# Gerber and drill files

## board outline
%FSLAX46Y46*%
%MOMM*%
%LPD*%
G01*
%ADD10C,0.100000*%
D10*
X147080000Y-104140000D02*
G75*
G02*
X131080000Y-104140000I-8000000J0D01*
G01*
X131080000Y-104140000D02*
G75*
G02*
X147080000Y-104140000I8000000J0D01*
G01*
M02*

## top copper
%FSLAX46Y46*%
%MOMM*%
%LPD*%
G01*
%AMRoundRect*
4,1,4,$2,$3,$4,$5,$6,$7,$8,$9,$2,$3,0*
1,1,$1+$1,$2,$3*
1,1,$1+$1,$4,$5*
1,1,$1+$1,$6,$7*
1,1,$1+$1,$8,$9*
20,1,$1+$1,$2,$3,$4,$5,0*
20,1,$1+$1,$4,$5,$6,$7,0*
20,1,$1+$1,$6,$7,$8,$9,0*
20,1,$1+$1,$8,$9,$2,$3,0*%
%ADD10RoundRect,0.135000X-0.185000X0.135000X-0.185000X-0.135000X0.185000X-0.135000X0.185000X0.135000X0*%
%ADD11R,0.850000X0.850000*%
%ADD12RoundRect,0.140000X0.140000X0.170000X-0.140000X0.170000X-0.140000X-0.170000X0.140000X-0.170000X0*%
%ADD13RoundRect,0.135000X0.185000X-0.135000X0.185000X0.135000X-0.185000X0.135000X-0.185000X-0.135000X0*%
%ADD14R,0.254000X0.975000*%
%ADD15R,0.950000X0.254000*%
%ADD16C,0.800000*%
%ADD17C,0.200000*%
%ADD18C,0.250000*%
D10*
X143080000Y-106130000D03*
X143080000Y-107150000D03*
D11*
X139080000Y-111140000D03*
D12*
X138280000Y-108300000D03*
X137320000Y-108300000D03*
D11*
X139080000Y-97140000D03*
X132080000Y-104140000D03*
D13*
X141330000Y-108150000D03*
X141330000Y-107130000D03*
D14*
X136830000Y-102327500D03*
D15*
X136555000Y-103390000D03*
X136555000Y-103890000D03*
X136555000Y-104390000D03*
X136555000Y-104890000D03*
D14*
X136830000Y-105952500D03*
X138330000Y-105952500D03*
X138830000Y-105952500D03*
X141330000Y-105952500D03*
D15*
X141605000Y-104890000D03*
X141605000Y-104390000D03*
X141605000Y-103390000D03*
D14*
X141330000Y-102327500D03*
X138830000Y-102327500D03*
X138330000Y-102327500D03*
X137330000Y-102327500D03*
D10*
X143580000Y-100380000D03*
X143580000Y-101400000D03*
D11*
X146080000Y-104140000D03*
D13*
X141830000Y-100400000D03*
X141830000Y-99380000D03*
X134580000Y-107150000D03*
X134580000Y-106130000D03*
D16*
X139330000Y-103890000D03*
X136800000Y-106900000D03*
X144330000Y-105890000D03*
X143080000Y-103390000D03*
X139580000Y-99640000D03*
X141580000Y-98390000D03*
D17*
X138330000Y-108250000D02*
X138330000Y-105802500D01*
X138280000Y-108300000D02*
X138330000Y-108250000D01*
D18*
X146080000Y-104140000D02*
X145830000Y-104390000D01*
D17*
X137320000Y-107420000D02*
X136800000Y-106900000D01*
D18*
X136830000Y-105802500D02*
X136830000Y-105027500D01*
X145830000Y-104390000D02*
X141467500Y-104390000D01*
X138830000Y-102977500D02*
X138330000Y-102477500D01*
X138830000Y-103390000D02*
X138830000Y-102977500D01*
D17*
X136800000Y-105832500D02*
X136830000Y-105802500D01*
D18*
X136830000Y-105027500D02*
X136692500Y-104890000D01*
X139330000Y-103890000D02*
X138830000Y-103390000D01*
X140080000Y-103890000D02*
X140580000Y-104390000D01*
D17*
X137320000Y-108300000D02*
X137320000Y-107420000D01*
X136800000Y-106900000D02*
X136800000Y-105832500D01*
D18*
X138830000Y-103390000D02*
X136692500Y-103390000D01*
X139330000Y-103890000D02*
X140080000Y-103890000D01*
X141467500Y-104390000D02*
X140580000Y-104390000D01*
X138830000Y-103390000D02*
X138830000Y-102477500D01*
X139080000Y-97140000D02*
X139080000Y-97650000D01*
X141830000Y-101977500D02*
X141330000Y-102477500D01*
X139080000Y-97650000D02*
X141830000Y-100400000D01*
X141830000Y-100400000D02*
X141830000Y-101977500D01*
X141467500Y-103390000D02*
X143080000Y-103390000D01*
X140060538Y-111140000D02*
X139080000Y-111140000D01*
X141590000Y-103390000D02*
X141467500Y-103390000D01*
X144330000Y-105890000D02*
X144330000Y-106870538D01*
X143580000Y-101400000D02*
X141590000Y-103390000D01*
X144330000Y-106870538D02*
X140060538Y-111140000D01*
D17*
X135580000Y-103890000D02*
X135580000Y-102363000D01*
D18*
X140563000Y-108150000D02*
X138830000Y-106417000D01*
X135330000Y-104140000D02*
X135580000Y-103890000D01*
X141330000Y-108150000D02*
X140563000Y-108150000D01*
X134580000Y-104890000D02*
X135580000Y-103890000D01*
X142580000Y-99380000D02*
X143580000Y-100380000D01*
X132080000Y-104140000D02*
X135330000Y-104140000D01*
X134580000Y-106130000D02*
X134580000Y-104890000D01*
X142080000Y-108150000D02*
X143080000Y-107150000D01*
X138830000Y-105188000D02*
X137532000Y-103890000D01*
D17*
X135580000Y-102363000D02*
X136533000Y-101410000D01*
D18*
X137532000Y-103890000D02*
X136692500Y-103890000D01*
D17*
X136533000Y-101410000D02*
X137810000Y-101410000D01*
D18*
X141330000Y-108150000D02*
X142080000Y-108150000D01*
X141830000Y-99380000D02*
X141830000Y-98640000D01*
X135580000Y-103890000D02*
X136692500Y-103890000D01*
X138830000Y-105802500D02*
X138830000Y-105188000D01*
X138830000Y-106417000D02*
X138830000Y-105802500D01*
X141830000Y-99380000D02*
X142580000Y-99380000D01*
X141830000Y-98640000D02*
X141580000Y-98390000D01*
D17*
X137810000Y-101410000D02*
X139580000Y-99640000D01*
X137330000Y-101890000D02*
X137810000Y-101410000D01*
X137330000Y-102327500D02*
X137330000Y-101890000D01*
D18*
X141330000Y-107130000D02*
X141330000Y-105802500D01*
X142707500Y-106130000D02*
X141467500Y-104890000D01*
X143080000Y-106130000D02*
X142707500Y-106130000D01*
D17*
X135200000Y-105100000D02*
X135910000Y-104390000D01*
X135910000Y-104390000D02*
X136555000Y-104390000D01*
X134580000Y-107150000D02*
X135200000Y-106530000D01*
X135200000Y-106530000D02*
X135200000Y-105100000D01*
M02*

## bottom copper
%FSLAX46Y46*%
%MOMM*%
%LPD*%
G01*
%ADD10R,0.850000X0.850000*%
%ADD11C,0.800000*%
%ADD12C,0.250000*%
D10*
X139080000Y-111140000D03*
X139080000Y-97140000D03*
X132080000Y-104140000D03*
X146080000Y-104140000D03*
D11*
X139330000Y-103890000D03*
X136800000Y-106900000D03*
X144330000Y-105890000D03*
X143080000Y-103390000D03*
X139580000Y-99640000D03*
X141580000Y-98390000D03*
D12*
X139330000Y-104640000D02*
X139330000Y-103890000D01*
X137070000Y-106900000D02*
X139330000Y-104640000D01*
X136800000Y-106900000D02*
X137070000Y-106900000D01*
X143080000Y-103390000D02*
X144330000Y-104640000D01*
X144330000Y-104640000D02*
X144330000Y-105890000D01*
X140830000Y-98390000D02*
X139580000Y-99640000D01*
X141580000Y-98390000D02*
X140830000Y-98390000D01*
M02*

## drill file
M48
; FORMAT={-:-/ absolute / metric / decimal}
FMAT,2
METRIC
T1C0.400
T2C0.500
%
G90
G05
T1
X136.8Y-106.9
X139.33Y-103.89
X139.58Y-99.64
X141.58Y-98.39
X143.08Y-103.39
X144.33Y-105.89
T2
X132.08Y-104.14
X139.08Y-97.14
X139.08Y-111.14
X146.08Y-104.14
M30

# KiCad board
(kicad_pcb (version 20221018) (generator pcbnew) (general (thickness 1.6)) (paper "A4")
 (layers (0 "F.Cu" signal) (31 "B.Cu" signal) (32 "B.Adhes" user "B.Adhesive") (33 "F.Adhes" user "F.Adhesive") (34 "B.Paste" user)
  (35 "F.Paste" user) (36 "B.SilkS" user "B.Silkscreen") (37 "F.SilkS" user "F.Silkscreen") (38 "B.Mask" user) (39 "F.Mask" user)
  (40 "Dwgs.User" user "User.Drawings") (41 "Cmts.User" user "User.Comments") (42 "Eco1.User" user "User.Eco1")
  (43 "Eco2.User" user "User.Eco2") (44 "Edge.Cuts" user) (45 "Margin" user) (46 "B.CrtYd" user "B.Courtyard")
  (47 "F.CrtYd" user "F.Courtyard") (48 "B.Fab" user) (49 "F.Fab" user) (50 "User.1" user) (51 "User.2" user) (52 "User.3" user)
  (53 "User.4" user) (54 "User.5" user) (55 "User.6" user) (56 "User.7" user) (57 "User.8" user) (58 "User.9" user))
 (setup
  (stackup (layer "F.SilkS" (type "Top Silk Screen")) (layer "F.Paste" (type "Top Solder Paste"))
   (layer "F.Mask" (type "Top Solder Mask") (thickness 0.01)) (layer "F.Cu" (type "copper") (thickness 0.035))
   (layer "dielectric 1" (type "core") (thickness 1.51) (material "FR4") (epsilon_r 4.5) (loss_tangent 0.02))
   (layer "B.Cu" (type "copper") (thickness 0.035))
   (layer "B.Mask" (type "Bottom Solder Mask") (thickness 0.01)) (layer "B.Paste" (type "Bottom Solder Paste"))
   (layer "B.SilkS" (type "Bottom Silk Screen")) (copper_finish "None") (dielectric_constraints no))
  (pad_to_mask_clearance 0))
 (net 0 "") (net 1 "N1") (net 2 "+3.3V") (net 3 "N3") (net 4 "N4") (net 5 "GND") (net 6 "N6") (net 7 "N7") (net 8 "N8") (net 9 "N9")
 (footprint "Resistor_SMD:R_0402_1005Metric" (layer "F.Cu") (at 143.08 106.64 -90)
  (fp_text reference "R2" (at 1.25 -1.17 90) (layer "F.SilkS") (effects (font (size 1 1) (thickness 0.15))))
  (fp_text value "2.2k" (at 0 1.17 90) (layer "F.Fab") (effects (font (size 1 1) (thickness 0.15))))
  (pad "1" smd roundrect (at -0.51 0 270) (size 0.54 0.64) (layers "F.Cu" "F.Paste" "F.Mask") (roundrect_rratio 0.25) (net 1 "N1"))
  (pad "2" smd roundrect (at 0.51 0 270) (size 0.54 0.64) (layers "F.Cu" "F.Paste" "F.Mask") (roundrect_rratio 0.25) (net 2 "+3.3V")))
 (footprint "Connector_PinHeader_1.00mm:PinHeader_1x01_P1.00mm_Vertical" (layer "F.Cu") (at 139.08 111.14 180)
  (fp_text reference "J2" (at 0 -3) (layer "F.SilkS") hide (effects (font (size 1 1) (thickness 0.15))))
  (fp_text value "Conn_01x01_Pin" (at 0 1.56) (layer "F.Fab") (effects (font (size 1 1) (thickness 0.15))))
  (pad "1" thru_hole rect (at 0 0 180) (size 0.85 0.85) (drill 0.5) (layers "*.Cu" "*.Mask") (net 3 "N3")))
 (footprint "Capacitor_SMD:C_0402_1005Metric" (layer "F.Cu") (at 137.8 108.3 180)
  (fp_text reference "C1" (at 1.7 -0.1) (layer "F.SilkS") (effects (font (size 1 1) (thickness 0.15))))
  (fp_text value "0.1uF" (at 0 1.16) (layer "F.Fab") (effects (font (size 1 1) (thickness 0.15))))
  (pad "1" smd roundrect (at -0.48 0 180) (size 0.56 0.62) (layers "F.Cu" "F.Paste" "F.Mask") (roundrect_rratio 0.25) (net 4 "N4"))
  (pad "2" smd roundrect (at 0.48 0 180) (size 0.56 0.62) (layers "F.Cu" "F.Paste" "F.Mask") (roundrect_rratio 0.25) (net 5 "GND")))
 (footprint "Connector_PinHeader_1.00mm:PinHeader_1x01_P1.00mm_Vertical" (layer "F.Cu") (at 139.08 97.14)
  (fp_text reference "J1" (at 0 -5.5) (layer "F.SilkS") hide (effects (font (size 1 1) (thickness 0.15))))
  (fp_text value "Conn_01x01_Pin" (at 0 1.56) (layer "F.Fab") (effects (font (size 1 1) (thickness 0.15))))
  (pad "1" thru_hole rect (at 0 0) (size 0.85 0.85) (drill 0.5) (layers "*.Cu" "*.Mask") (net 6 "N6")))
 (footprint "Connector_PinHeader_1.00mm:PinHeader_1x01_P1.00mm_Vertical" (layer "F.Cu") (at 132.08 104.14 90)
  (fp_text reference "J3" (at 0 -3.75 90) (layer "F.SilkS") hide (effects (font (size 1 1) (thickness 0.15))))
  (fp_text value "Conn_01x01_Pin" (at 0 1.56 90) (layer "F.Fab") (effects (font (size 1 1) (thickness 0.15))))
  (pad "1" thru_hole rect (at 0 0 90) (size 0.85 0.85) (drill 0.5) (layers "*.Cu" "*.Mask") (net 2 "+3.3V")))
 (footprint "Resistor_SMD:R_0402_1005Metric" (layer "F.Cu") (at 141.33 107.64 90)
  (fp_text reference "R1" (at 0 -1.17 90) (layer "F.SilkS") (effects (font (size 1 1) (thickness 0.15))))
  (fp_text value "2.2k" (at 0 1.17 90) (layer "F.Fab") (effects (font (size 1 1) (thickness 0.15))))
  (pad "1" smd roundrect (at -0.51 0 90) (size 0.54 0.64) (layers "F.Cu" "F.Paste" "F.Mask") (roundrect_rratio 0.25) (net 2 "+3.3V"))
  (pad "2" smd roundrect (at 0.51 0 90) (size 0.54 0.64) (layers "F.Cu" "F.Paste" "F.Mask") (roundrect_rratio 0.25) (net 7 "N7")))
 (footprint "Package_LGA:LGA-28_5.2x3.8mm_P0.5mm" (layer "F.Cu") (at 139.08 104.14)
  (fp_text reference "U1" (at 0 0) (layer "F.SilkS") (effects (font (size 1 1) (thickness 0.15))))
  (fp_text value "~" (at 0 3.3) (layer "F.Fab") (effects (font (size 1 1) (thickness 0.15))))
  (pad "1" smd rect (at -2.25 -1.8125) (size 0.254 0.975) (layers "F.Cu" "F.Paste" "F.Mask") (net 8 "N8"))
  (pad "2" smd rect (at -2.525 -0.75 90) (size 0.254 0.95) (layers "F.Cu" "F.Paste" "F.Mask") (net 5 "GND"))
  (pad "3" smd rect (at -2.525 -0.25 90) (size 0.254 0.95) (layers "F.Cu" "F.Paste" "F.Mask") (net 2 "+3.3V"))
  (pad "4" smd rect (at -2.525 0.25 90) (size 0.254 0.95) (layers "F.Cu" "F.Paste" "F.Mask") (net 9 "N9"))
  (pad "5" smd rect (at -2.525 0.75 90) (size 0.254 0.95) (layers "F.Cu" "F.Paste" "F.Mask") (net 5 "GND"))
  (pad "6" smd rect (at -2.25 1.8125) (size 0.254 0.975) (layers "F.Cu" "F.Paste" "F.Mask") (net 5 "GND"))
  (pad "9" smd rect (at -0.75 1.8125) (size 0.254 0.975) (layers "F.Cu" "F.Paste" "F.Mask") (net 4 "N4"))
  (pad "10" smd rect (at -0.25 1.8125) (size 0.254 0.975) (layers "F.Cu" "F.Paste" "F.Mask") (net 2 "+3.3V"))
  (pad "15" smd rect (at 2.25 1.8125) (size 0.254 0.975) (layers "F.Cu" "F.Paste" "F.Mask") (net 7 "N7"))
  (pad "16" smd rect (at 2.525 0.75 90) (size 0.254 0.95) (layers "F.Cu" "F.Paste" "F.Mask") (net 1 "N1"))
  (pad "17" smd rect (at 2.525 0.25 90) (size 0.254 0.95) (layers "F.Cu" "F.Paste" "F.Mask") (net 5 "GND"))
  (pad "19" smd rect (at 2.525 -0.75 90) (size 0.254 0.95) (layers "F.Cu" "F.Paste" "F.Mask") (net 3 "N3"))
  (pad "20" smd rect (at 2.25 -1.8125) (size 0.254 0.975) (layers "F.Cu" "F.Paste" "F.Mask") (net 6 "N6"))
  (pad "25" smd rect (at -0.25 -1.8125) (size 0.254 0.975) (layers "F.Cu" "F.Paste" "F.Mask") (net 5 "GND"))
  (pad "26" smd rect (at -0.75 -1.8125) (size 0.254 0.975) (layers "F.Cu" "F.Paste" "F.Mask") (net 5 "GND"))
  (pad "28" smd rect (at -1.75 -1.8125) (size 0.254 0.975) (layers "F.Cu" "F.Paste" "F.Mask") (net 2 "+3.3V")))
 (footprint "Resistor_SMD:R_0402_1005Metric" (layer "F.Cu") (at 143.58 100.89 -90)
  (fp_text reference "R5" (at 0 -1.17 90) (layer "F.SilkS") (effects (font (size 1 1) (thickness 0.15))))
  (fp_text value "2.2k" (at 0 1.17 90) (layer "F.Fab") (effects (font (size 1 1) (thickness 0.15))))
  (pad "1" smd roundrect (at -0.51 0 270) (size 0.54 0.64) (layers "F.Cu" "F.Paste" "F.Mask") (roundrect_rratio 0.25) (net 2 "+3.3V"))
  (pad "2" smd roundrect (at 0.51 0 270) (size 0.54 0.64) (layers "F.Cu" "F.Paste" "F.Mask") (roundrect_rratio 0.25) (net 3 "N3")))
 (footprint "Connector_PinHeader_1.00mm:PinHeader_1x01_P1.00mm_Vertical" (layer "F.Cu") (at 146.08 104.14 -90)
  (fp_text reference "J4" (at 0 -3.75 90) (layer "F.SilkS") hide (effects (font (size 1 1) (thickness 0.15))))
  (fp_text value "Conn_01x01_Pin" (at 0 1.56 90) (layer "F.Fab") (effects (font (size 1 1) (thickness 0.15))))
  (pad "1" thru_hole rect (at 0 0 270) (size 0.85 0.85) (drill 0.5) (layers "*.Cu" "*.Mask") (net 5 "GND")))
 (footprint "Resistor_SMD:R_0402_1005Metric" (layer "F.Cu") (at 141.83 99.89 90)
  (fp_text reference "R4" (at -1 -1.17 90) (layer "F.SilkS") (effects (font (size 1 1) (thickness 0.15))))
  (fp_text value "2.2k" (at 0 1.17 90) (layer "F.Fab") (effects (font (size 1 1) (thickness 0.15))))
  (pad "1" smd roundrect (at -0.51 0 90) (size 0.54 0.64) (layers "F.Cu" "F.Paste" "F.Mask") (roundrect_rratio 0.25) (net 6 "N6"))
  (pad "2" smd roundrect (at 0.51 0 90) (size 0.54 0.64) (layers "F.Cu" "F.Paste" "F.Mask") (roundrect_rratio 0.25) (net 2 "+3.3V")))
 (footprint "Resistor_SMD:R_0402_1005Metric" (layer "F.Cu") (at 134.58 106.64 90)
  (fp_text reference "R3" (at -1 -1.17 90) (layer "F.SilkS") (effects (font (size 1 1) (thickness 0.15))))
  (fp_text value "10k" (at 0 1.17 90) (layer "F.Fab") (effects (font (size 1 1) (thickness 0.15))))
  (pad "1" smd roundrect (at -0.51 0 90) (size 0.54 0.64) (layers "F.Cu" "F.Paste" "F.Mask") (roundrect_rratio 0.25) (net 9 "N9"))
  (pad "2" smd roundrect (at 0.51 0 90) (size 0.54 0.64) (layers "F.Cu" "F.Paste" "F.Mask") (roundrect_rratio 0.25) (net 2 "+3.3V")))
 (gr_circle (center 139.08 104.14) (end 147.08 104.14) (stroke (width 0.1) (type default)) (fill none) (layer "Edge.Cuts"))
 (segment (start 138.33 108.25) (end 138.33 105.8025) (width 0.2) (layer "F.Cu") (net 4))
 (segment (start 138.28 108.3) (end 138.33 108.25) (width 0.2) (layer "F.Cu") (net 4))
 (segment (start 146.08 104.14) (end 145.83 104.39) (width 0.25) (layer "F.Cu") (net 5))
 (segment (start 137.32 107.42) (end 136.8 106.9) (width 0.2) (layer "F.Cu") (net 5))
 (segment (start 136.83 105.8025) (end 136.83 105.0275) (width 0.25) (layer "F.Cu") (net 5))
 (segment (start 145.83 104.39) (end 141.4675 104.39) (width 0.25) (layer "F.Cu") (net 5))
 (segment (start 138.83 102.9775) (end 138.33 102.4775) (width 0.25) (layer "F.Cu") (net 5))
 (segment (start 138.83 103.39) (end 138.83 102.9775) (width 0.25) (layer "F.Cu") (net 5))
 (segment (start 136.8 105.8325) (end 136.83 105.8025) (width 0.2) (layer "F.Cu") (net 5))
 (segment (start 136.83 105.0275) (end 136.6925 104.89) (width 0.25) (layer "F.Cu") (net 5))
 (segment (start 139.33 103.89) (end 138.83 103.39) (width 0.25) (layer "F.Cu") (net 5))
 (segment (start 140.08 103.89) (end 140.58 104.39) (width 0.25) (layer "F.Cu") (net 5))
 (segment (start 137.32 108.3) (end 137.32 107.42) (width 0.2) (layer "F.Cu") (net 5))
 (segment (start 136.8 106.9) (end 136.8 105.8325) (width 0.2) (layer "F.Cu") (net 5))
 (segment (start 138.83 103.39) (end 136.6925 103.39) (width 0.25) (layer "F.Cu") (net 5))
 (segment (start 139.33 103.89) (end 140.08 103.89) (width 0.25) (layer "F.Cu") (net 5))
 (segment (start 141.4675 104.39) (end 140.58 104.39) (width 0.25) (layer "F.Cu") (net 5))
 (segment (start 138.83 103.39) (end 138.83 102.4775) (width 0.25) (layer "F.Cu") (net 5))
 (via (at 139.33 103.89) (size 0.8) (drill 0.4) (layers "F.Cu" "B.Cu") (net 5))
 (via (at 136.8 106.9) (size 0.8) (drill 0.4) (layers "F.Cu" "B.Cu") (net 5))
 (segment (start 139.33 104.64) (end 139.33 103.89) (width 0.25) (layer "B.Cu") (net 5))
 (segment (start 137.07 106.9) (end 139.33 104.64) (width 0.25) (layer "B.Cu") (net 5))
 (segment (start 136.8 106.9) (end 137.07 106.9) (width 0.25) (layer "B.Cu") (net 5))
 (segment (start 139.08 97.14) (end 139.08 97.65) (width 0.25) (layer "F.Cu") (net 6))
 (segment (start 141.83 101.9775) (end 141.33 102.4775) (width 0.25) (layer "F.Cu") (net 6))
 (segment (start 139.08 97.65) (end 141.83 100.4) (width 0.25) (layer "F.Cu") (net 6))
 (segment (start 141.83 100.4) (end 141.83 101.9775) (width 0.25) (layer "F.Cu") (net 6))
 (segment (start 141.4675 103.39) (end 143.08 103.39) (width 0.25) (layer "F.Cu") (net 3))
 (segment (start 140.060538 111.14) (end 139.08 111.14) (width 0.25) (layer "F.Cu") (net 3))
 (segment (start 141.59 103.39) (end 141.4675 103.39) (width 0.25) (layer "F.Cu") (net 3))
 (segment (start 144.33 105.89) (end 144.33 106.870538) (width 0.25) (layer "F.Cu") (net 3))
 (segment (start 143.58 101.4) (end 141.59 103.39) (width 0.25) (layer "F.Cu") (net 3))
 (segment (start 144.33 106.870538) (end 140.060538 111.14) (width 0.25) (layer "F.Cu") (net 3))
 (via (at 144.33 105.89) (size 0.8) (drill 0.4) (layers "F.Cu" "B.Cu") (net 3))
 (via (at 143.08 103.39) (size 0.8) (drill 0.4) (layers "F.Cu" "B.Cu") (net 3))
 (segment (start 143.08 103.39) (end 144.33 104.64) (width 0.25) (layer "B.Cu") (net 3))
 (segment (start 144.33 104.64) (end 144.33 105.89) (width 0.25) (layer "B.Cu") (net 3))
 (segment (start 135.58 103.89) (end 135.58 102.363) (width 0.2) (layer "F.Cu") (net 2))
 (segment (start 140.563 108.15) (end 138.83 106.417) (width 0.25) (layer "F.Cu") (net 2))
 (segment (start 135.33 104.14) (end 135.58 103.89) (width 0.25) (layer "F.Cu") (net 2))
 (segment (start 141.33 108.15) (end 140.563 108.15) (width 0.25) (layer "F.Cu") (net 2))
 (segment (start 134.58 104.89) (end 135.58 103.89) (width 0.25) (layer "F.Cu") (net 2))
 (segment (start 142.58 99.38) (end 143.58 100.38) (width 0.25) (layer "F.Cu") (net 2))
 (segment (start 132.08 104.14) (end 135.33 104.14) (width 0.25) (layer "F.Cu") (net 2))
 (segment (start 134.58 106.13) (end 134.58 104.89) (width 0.25) (layer "F.Cu") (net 2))
 (segment (start 142.08 108.15) (end 143.08 107.15) (width 0.25) (layer "F.Cu") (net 2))
 (segment (start 138.83 105.188) (end 137.532 103.89) (width 0.25) (layer "F.Cu") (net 2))
 (segment (start 135.58 102.363) (end 136.533 101.41) (width 0.2) (layer "F.Cu") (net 2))
 (segment (start 137.532 103.89) (end 136.6925 103.89) (width 0.25) (layer "F.Cu") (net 2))
 (segment (start 136.533 101.41) (end 137.81 101.41) (width 0.2) (layer "F.Cu") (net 2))
 (segment (start 141.33 108.15) (end 142.08 108.15) (width 0.25) (layer "F.Cu") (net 2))
 (segment (start 141.83 99.38) (end 141.83 98.64) (width 0.25) (layer "F.Cu") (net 2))
 (segment (start 135.58 103.89) (end 136.6925 103.89) (width 0.25) (layer "F.Cu") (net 2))
 (segment (start 138.83 105.8025) (end 138.83 105.188) (width 0.25) (layer "F.Cu") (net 2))
 (segment (start 138.83 106.417) (end 138.83 105.8025) (width 0.25) (layer "F.Cu") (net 2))
 (segment (start 141.83 99.38) (end 142.58 99.38) (width 0.25) (layer "F.Cu") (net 2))
 (segment (start 141.83 98.64) (end 141.58 98.39) (width 0.25) (layer "F.Cu") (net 2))
 (segment (start 137.81 101.41) (end 139.58 99.64) (width 0.2) (layer "F.Cu") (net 2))
 (segment (start 137.33 101.89) (end 137.81 101.41) (width 0.2) (layer "F.Cu") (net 2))
 (segment (start 137.33 102.3275) (end 137.33 101.89) (width 0.2) (layer "F.Cu") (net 2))
 (via (at 139.58 99.64) (size 0.8) (drill 0.4) (layers "F.Cu" "B.Cu") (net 2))
 (via (at 141.58 98.39) (size 0.8) (drill 0.4) (layers "F.Cu" "B.Cu") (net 2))
 (segment (start 140.83 98.39) (end 139.58 99.64) (width 0.25) (layer "B.Cu") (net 2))
 (segment (start 141.58 98.39) (end 140.83 98.39) (width 0.25) (layer "B.Cu") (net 2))
 (segment (start 141.33 107.13) (end 141.33 105.8025) (width 0.25) (layer "F.Cu") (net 7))
 (segment (start 142.7075 106.13) (end 141.4675 104.89) (width 0.25) (layer "F.Cu") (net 1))
 (segment (start 143.08 106.13) (end 142.7075 106.13) (width 0.25) (layer "F.Cu") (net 1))
 (segment (start 135.2 105.1) (end 135.91 104.39) (width 0.2) (layer "F.Cu") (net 9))
 (segment (start 135.91 104.39) (end 136.555 104.39) (width 0.2) (layer "F.Cu") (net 9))
 (segment (start 134.58 107.15) (end 135.2 106.53) (width 0.2) (layer "F.Cu") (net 9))
 (segment (start 135.2 106.53) (end 135.2 105.1) (width 0.2) (layer "F.Cu") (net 9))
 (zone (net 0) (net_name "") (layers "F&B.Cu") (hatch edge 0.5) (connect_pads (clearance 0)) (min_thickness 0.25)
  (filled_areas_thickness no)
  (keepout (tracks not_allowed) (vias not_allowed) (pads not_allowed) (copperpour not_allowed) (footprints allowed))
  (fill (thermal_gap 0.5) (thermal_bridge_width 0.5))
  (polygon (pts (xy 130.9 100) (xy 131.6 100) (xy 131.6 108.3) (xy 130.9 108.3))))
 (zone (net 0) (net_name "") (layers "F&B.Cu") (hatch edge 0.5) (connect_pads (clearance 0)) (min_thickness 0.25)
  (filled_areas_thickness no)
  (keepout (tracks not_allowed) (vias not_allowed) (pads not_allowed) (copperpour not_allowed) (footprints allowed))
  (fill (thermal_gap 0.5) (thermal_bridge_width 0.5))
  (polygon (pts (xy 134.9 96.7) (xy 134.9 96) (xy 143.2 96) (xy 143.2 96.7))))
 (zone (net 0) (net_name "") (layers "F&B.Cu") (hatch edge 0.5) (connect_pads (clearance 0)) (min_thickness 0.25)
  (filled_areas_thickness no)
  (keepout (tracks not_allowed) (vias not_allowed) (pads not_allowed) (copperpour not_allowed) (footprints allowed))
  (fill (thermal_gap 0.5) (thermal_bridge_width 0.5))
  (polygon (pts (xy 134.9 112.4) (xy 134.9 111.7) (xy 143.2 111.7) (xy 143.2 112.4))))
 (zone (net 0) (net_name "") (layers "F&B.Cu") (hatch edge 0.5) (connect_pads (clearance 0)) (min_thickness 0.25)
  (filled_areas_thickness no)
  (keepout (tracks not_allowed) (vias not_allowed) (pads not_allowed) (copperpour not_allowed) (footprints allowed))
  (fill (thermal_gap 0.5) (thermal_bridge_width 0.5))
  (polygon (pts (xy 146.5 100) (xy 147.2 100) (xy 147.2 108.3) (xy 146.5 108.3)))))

